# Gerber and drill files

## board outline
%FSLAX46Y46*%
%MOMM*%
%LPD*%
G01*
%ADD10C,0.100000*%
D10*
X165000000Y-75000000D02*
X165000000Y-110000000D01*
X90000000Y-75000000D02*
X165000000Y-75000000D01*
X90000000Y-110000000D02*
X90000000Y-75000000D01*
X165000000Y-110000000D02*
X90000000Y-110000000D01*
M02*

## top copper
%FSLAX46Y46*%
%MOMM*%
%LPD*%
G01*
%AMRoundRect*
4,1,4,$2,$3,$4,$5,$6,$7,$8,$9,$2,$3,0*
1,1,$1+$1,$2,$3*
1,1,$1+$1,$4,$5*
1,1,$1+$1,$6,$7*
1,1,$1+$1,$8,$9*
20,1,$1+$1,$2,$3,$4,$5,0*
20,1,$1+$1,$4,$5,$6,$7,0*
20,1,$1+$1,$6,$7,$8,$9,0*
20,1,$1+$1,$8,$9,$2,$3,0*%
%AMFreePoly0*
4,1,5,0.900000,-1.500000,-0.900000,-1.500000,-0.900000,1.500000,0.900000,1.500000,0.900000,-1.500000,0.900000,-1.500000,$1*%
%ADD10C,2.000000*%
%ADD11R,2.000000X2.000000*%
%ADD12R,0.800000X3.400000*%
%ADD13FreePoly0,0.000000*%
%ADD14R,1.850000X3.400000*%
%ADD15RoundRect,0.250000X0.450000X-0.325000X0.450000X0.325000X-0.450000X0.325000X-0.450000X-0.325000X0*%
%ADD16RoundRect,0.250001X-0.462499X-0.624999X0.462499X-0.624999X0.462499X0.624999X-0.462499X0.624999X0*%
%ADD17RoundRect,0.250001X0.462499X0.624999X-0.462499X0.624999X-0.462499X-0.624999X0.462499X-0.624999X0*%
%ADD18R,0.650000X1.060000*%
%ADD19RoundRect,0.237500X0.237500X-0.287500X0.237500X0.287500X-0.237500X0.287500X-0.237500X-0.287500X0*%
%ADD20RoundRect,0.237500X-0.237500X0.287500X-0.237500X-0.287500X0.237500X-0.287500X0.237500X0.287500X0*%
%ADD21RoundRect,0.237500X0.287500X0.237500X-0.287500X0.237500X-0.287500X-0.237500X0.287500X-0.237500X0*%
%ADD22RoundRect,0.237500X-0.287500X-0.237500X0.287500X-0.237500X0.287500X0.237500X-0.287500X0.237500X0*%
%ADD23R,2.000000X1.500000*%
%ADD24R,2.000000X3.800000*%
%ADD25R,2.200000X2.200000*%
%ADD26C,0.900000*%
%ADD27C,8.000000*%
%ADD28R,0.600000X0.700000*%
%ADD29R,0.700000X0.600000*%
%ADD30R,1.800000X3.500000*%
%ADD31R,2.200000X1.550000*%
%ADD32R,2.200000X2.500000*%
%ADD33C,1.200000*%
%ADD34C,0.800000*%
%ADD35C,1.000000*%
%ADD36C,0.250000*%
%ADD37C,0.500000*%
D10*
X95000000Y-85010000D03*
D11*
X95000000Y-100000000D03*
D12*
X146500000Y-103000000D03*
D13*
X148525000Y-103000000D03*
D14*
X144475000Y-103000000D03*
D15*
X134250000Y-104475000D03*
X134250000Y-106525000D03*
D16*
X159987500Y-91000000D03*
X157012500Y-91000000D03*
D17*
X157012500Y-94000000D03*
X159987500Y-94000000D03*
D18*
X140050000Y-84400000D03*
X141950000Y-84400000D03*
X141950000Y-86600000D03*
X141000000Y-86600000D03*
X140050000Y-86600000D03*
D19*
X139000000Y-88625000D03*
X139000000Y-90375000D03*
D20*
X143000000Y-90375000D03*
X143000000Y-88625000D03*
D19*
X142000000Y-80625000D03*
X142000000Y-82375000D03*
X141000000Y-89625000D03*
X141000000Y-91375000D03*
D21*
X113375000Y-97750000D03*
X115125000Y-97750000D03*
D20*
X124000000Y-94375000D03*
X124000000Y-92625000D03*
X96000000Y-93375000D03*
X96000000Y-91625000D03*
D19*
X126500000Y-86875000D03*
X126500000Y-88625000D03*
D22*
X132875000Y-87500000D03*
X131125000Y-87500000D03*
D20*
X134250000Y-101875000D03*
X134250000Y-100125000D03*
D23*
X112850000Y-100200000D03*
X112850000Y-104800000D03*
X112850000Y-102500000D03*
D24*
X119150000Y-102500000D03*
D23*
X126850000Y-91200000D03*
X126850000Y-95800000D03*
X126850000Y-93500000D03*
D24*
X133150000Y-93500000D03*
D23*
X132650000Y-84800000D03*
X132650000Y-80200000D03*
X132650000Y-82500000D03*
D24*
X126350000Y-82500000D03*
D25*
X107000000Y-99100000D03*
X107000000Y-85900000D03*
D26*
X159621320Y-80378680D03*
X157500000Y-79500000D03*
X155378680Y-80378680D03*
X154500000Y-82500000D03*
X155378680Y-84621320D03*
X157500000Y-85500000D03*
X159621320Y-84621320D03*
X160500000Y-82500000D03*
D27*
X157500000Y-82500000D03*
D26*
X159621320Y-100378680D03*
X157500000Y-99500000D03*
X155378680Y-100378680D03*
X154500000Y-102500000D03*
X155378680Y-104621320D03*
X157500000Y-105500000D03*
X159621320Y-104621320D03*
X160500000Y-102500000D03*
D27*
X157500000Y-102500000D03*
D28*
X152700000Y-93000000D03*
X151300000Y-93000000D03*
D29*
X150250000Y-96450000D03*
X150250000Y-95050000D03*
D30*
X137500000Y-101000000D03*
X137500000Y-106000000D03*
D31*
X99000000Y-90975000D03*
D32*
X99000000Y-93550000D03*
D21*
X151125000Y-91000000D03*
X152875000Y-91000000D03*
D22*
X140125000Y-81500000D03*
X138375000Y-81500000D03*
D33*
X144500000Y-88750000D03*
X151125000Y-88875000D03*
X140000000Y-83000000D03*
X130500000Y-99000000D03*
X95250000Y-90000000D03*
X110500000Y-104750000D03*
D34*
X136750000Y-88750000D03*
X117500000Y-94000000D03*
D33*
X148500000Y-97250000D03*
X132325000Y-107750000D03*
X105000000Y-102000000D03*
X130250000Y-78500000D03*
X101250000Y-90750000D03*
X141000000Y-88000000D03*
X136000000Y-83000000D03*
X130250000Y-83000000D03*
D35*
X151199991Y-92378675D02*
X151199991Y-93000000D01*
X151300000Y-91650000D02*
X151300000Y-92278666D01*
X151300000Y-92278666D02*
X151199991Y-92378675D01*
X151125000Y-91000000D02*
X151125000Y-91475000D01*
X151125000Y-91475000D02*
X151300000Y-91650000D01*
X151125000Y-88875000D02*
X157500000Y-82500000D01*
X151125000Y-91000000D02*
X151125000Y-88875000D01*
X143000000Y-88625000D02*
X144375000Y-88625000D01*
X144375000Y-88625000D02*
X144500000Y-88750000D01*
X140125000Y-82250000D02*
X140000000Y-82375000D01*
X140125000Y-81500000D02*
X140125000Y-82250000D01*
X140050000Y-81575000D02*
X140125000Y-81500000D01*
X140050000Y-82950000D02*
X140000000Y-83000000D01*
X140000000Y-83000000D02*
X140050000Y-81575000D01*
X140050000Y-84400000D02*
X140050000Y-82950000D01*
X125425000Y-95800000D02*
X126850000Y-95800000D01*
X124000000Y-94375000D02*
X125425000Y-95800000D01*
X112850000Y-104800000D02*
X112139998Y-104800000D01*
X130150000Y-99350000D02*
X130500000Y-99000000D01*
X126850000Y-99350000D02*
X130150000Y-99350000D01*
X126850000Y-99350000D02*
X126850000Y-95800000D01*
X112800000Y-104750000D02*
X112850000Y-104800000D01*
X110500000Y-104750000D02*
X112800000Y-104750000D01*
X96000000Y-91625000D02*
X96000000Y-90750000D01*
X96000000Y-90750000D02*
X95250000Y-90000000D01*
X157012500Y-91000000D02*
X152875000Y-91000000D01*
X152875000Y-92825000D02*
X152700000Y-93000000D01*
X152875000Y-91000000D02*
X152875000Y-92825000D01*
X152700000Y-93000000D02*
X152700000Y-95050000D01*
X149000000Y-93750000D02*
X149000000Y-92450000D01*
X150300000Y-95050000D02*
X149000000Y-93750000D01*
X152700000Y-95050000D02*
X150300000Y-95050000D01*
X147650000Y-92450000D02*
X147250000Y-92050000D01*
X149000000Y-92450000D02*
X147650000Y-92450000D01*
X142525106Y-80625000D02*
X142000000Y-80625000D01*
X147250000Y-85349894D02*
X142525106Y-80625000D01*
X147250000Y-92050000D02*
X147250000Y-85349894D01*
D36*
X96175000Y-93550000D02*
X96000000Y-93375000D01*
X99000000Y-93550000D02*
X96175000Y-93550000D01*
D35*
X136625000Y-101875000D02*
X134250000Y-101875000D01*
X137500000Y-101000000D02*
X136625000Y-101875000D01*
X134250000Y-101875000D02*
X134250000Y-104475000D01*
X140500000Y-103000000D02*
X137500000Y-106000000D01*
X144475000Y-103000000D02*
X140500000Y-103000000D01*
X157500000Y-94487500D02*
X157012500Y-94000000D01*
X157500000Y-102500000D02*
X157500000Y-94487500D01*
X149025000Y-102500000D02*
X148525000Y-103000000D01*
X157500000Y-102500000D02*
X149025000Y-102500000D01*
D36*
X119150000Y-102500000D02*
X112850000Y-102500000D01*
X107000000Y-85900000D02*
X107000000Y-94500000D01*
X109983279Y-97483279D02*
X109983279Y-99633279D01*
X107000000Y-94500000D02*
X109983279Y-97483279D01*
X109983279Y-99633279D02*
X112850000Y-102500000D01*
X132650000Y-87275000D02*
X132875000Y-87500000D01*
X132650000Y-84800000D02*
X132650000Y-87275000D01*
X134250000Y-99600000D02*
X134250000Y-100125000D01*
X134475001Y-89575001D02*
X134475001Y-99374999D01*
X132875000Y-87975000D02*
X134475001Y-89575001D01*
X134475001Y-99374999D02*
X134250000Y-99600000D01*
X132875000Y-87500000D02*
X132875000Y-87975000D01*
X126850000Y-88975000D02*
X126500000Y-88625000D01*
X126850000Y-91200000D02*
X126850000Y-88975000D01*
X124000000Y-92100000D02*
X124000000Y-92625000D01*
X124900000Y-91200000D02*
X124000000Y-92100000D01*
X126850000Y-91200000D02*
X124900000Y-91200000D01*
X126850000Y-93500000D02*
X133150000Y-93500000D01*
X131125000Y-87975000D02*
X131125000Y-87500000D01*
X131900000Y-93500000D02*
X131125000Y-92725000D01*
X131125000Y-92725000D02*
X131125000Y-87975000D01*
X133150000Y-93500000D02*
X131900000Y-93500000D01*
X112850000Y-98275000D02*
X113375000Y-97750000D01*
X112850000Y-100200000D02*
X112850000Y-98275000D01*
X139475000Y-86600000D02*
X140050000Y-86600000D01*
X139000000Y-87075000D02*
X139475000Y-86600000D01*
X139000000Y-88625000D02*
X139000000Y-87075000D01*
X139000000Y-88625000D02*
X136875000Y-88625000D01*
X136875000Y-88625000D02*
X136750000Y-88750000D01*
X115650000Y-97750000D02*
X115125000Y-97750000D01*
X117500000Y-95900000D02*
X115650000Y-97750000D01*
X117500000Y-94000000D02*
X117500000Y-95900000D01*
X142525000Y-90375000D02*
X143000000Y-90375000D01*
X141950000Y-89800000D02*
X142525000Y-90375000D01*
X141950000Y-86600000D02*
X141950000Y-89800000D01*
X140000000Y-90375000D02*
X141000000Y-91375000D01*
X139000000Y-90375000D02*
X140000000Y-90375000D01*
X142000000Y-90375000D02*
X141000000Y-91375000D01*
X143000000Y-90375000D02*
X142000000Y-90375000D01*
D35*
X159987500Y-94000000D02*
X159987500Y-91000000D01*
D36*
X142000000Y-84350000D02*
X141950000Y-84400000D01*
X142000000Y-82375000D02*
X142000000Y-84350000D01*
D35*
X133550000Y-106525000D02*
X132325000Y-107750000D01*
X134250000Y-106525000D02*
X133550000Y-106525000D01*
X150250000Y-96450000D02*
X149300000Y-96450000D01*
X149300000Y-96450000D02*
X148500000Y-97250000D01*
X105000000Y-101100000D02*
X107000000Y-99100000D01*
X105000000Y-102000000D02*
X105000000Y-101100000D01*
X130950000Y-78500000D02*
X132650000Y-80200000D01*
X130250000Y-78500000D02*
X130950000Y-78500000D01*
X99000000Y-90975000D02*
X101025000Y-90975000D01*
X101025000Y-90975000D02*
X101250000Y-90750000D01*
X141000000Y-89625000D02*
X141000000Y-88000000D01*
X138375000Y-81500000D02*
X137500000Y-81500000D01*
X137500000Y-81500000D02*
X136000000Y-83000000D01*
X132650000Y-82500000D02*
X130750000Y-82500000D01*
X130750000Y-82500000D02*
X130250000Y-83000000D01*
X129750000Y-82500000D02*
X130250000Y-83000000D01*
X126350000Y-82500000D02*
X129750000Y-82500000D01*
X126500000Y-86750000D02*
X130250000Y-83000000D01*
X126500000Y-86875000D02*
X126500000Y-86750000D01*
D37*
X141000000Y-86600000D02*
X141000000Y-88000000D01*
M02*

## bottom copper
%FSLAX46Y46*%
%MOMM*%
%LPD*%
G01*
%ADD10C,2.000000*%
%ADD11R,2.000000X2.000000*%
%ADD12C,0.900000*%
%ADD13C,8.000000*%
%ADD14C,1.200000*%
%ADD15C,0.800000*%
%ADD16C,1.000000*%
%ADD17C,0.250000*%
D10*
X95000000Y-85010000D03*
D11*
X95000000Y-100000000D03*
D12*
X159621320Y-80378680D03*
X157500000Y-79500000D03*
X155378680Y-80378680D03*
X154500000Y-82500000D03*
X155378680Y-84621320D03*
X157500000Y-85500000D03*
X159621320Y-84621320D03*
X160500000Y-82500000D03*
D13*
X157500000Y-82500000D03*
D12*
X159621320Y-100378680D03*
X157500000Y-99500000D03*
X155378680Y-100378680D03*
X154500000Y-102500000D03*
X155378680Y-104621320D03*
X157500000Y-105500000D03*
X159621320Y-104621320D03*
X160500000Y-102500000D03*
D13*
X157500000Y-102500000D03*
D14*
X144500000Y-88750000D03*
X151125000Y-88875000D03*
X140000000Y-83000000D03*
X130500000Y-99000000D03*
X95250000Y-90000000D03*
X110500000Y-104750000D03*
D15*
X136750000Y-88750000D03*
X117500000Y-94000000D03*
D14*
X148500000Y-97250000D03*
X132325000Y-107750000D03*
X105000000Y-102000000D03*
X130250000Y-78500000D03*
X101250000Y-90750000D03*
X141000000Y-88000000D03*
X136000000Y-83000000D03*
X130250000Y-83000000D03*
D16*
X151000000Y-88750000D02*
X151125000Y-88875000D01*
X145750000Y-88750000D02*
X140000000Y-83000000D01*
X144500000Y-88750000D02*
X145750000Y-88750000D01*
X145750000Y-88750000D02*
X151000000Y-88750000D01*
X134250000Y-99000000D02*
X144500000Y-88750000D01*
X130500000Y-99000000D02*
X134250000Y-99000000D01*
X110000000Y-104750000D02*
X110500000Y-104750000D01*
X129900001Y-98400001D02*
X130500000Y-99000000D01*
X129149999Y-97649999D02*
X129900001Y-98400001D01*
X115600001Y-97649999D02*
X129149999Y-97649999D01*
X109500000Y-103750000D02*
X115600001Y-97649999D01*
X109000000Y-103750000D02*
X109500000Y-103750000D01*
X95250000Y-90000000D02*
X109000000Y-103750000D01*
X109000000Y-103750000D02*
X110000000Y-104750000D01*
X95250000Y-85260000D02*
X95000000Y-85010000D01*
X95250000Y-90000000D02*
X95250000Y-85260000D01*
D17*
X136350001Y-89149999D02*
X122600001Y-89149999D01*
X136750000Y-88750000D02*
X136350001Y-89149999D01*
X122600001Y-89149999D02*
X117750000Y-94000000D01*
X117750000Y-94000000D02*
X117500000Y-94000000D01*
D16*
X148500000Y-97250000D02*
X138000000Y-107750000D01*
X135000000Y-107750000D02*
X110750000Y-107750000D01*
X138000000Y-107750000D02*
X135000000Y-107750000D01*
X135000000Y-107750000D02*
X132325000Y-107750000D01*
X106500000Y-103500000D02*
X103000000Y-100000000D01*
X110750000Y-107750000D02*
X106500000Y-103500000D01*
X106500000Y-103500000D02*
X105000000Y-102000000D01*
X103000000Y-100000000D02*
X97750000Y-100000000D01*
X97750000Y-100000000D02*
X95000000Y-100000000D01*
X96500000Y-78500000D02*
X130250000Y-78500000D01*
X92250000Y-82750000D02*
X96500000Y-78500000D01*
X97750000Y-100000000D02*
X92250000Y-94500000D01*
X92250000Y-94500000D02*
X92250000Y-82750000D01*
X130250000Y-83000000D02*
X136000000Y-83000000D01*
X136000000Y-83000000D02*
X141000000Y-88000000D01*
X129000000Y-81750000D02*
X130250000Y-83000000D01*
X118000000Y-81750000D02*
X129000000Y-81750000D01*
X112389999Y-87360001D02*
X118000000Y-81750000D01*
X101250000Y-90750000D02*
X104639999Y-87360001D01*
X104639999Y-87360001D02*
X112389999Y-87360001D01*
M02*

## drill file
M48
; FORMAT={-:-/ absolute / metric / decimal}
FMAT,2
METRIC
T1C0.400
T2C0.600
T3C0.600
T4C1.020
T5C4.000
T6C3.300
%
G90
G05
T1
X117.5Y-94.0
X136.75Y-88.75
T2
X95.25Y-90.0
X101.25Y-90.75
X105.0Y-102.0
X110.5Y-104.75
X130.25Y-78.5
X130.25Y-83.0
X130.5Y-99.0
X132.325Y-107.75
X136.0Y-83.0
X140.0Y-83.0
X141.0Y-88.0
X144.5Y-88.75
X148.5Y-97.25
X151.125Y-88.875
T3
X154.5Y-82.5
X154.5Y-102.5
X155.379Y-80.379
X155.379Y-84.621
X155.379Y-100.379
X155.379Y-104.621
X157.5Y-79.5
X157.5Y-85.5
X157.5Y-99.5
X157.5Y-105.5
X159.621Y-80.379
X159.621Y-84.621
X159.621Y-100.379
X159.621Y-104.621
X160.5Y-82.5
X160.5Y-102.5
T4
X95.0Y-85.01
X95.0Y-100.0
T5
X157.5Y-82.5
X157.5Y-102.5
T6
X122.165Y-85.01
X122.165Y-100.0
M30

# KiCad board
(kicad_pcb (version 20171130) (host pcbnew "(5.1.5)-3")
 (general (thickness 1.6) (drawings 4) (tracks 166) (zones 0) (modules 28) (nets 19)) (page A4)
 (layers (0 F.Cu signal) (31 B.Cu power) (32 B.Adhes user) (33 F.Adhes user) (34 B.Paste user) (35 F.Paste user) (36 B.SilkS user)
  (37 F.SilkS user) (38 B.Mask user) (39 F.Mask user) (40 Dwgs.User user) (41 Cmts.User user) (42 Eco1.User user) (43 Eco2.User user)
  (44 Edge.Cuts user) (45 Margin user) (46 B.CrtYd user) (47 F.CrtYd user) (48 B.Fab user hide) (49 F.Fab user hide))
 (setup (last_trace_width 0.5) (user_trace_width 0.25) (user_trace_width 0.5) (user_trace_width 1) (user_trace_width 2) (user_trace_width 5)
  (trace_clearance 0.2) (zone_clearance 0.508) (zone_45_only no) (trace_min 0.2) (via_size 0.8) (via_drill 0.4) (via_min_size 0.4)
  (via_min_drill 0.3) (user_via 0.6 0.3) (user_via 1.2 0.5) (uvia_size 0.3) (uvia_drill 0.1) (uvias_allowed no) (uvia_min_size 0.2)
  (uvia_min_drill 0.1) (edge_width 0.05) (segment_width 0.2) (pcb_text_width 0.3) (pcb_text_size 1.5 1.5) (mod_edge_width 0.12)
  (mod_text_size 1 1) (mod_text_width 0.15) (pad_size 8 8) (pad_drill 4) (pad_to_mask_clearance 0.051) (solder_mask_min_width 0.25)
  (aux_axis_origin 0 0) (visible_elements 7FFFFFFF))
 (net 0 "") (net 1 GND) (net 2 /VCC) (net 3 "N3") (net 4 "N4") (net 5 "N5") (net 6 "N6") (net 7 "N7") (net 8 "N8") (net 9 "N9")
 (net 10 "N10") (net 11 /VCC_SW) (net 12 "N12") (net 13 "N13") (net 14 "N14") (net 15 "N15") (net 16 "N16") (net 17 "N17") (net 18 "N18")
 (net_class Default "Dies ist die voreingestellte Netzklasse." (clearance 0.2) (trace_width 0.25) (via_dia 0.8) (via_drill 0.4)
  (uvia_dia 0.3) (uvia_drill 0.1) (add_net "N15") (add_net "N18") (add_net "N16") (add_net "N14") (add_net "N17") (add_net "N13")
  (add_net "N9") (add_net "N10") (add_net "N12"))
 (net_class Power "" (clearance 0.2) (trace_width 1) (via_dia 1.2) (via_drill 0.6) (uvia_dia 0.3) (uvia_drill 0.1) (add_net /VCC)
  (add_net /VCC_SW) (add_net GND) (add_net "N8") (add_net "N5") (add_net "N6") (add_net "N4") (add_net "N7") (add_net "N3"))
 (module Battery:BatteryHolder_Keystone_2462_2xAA (layer B.Cu) (at 95 100)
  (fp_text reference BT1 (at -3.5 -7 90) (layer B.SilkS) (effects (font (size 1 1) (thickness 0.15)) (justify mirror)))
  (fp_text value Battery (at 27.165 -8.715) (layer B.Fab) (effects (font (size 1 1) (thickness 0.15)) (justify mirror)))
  (pad "" np_thru_hole circle (at 27.165 0) (size 3.3 3.3) (drill 3.3) (layers *.Cu *.Mask))
  (pad "" np_thru_hole circle (at 27.165 -14.99) (size 3.3 3.3) (drill 3.3) (layers *.Cu *.Mask))
  (pad 2 thru_hole circle (at 0 -14.99) (size 2 2) (drill 1.02) (layers *.Cu *.Mask) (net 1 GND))
  (pad 1 thru_hole rect (at 0 0) (size 2 2) (drill 1.02) (layers *.Cu *.Mask) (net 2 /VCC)))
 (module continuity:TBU (layer F.Cu) (at 146.5 103)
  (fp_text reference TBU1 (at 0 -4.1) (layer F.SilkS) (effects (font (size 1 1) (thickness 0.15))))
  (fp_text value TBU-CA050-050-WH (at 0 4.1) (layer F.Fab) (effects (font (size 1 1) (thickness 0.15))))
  (pad 2 smd rect (at 0 0) (size 0.8 3.4) (layers F.Cu F.Paste F.Mask) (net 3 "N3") (zone_connect 2))
  (pad 3 smd custom (at 2.025 0) (size 1.8 3) (layers F.Cu F.Paste F.Mask) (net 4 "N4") (zone_connect 2)
   (options (clearance outline) (anchor rect)) (primitives))
  (pad 1 smd rect (at -2.025 0) (size 1.85 3.4) (layers F.Cu F.Paste F.Mask) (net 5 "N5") (zone_connect 2)))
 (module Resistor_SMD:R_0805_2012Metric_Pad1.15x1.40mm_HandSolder (layer F.Cu) (at 134.25 105.5 90)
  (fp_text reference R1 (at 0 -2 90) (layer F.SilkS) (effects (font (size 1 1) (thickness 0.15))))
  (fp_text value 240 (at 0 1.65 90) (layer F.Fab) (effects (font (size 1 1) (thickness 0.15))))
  (pad 2 smd roundrect (at 1.025 0 90) (size 1.15 1.4) (layers F.Cu F.Paste F.Mask) (roundrect_rratio 0.217391) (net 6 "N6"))
  (pad 1 smd roundrect (at -1.025 0 90) (size 1.15 1.4) (layers F.Cu F.Paste F.Mask) (roundrect_rratio 0.217391) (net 2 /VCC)))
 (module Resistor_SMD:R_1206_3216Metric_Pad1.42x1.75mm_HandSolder (layer F.Cu) (at 158.5 91)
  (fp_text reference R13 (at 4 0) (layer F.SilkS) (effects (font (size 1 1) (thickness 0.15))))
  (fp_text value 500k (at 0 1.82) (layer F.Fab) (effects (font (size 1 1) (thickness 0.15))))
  (pad 2 smd roundrect (at 1.4875 0) (size 1.425 1.75) (layers F.Cu F.Paste F.Mask) (roundrect_rratio 0.175439) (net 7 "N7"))
  (pad 1 smd roundrect (at -1.4875 0) (size 1.425 1.75) (layers F.Cu F.Paste F.Mask) (roundrect_rratio 0.175439) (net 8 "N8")))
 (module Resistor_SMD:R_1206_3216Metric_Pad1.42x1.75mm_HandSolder (layer F.Cu) (at 158.5 94 180)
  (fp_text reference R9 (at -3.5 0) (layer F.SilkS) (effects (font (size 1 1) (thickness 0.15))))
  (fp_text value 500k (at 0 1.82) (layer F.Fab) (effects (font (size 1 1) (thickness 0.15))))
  (pad 2 smd roundrect (at 1.4875 0 180) (size 1.425 1.75) (layers F.Cu F.Paste F.Mask) (roundrect_rratio 0.175439) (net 4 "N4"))
  (pad 1 smd roundrect (at -1.4875 0 180) (size 1.425 1.75) (layers F.Cu F.Paste F.Mask) (roundrect_rratio 0.175439) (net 7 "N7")))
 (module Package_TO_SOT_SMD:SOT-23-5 (layer F.Cu) (at 141 85.5 90)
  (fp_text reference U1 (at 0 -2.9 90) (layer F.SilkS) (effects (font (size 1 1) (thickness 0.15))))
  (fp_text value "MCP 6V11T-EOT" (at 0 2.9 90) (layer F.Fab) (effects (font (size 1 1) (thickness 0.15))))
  (pad 5 smd rect (at 1.1 -0.95 90) (size 1.06 0.65) (layers F.Cu F.Paste F.Mask) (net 1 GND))
  (pad 4 smd rect (at 1.1 0.95 90) (size 1.06 0.65) (layers F.Cu F.Paste F.Mask) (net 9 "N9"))
  (pad 3 smd rect (at -1.1 0.95 90) (size 1.06 0.65) (layers F.Cu F.Paste F.Mask) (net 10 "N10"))
  (pad 2 smd rect (at -1.1 0 90) (size 1.06 0.65) (layers F.Cu F.Paste F.Mask) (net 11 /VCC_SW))
  (pad 1 smd rect (at -1.1 -0.95 90) (size 1.06 0.65) (layers F.Cu F.Paste F.Mask) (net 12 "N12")))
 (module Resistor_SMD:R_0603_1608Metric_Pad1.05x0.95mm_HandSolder (layer F.Cu) (at 139 89.5 90)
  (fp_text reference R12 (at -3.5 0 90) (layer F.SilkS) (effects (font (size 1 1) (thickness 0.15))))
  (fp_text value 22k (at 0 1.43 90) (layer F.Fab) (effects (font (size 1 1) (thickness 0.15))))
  (pad 2 smd roundrect (at 0.875 0 90) (size 1.05 0.95) (layers F.Cu F.Paste F.Mask) (roundrect_rratio 0.25) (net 12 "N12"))
  (pad 1 smd roundrect (at -0.875 0 90) (size 1.05 0.95) (layers F.Cu F.Paste F.Mask) (roundrect_rratio 0.25) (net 10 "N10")))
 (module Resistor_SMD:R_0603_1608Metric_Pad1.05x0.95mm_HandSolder (layer F.Cu) (at 143 89.5 270)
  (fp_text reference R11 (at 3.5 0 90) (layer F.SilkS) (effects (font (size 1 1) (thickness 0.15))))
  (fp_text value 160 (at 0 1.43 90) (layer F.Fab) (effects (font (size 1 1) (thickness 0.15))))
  (pad 2 smd roundrect (at 0.875 0 270) (size 1.05 0.95) (layers F.Cu F.Paste F.Mask) (roundrect_rratio 0.25) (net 10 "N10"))
  (pad 1 smd roundrect (at -0.875 0 270) (size 1.05 0.95) (layers F.Cu F.Paste F.Mask) (roundrect_rratio 0.25) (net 1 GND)))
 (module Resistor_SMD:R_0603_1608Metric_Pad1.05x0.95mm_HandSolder (layer F.Cu) (at 142 81.5 90)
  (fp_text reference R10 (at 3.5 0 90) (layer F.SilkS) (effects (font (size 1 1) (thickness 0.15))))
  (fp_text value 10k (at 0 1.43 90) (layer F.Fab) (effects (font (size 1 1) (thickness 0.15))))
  (pad 2 smd roundrect (at 0.875 0 90) (size 1.05 0.95) (layers F.Cu F.Paste F.Mask) (roundrect_rratio 0.25) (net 8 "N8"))
  (pad 1 smd roundrect (at -0.875 0 90) (size 1.05 0.95) (layers F.Cu F.Paste F.Mask) (roundrect_rratio 0.25) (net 9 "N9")))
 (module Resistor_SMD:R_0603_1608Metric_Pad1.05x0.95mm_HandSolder (layer F.Cu) (at 141 90.5 90)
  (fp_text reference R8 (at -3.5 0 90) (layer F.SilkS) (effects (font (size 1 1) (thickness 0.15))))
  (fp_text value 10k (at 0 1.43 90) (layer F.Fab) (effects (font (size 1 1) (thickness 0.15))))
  (pad 2 smd roundrect (at 0.875 0 90) (size 1.05 0.95) (layers F.Cu F.Paste F.Mask) (roundrect_rratio 0.25) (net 11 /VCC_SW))
  (pad 1 smd roundrect (at -0.875 0 90) (size 1.05 0.95) (layers F.Cu F.Paste F.Mask) (roundrect_rratio 0.25) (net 10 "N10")))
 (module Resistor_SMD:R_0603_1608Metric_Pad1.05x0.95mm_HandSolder (layer F.Cu) (at 114.25 97.75 180)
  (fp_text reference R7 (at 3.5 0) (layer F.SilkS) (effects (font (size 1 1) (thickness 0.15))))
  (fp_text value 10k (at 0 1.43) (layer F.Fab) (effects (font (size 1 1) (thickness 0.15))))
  (pad 2 smd roundrect (at 0.875 0 180) (size 1.05 0.95) (layers F.Cu F.Paste F.Mask) (roundrect_rratio 0.25) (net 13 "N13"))
  (pad 1 smd roundrect (at -0.875 0 180) (size 1.05 0.95) (layers F.Cu F.Paste F.Mask) (roundrect_rratio 0.25) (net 12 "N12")))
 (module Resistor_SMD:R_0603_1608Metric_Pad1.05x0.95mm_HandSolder (layer F.Cu) (at 124 93.5 270)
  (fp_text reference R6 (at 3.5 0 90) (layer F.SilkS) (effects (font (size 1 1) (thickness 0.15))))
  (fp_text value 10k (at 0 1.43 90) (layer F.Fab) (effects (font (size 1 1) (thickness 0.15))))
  (pad 2 smd roundrect (at 0.875 0 270) (size 1.05 0.95) (layers F.Cu F.Paste F.Mask) (roundrect_rratio 0.25) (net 1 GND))
  (pad 1 smd roundrect (at -0.875 0 270) (size 1.05 0.95) (layers F.Cu F.Paste F.Mask) (roundrect_rratio 0.25) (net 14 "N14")))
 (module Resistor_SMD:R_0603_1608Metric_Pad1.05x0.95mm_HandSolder (layer F.Cu) (at 96 92.5 270)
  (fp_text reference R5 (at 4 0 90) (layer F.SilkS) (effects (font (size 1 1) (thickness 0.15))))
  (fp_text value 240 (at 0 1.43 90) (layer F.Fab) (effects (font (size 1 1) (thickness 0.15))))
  (pad 2 smd roundrect (at 0.875 0 270) (size 1.05 0.95) (layers F.Cu F.Paste F.Mask) (roundrect_rratio 0.25) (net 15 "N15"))
  (pad 1 smd roundrect (at -0.875 0 270) (size 1.05 0.95) (layers F.Cu F.Paste F.Mask) (roundrect_rratio 0.25) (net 1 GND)))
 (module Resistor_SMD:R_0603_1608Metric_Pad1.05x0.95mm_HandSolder (layer F.Cu) (at 126.5 87.75 90)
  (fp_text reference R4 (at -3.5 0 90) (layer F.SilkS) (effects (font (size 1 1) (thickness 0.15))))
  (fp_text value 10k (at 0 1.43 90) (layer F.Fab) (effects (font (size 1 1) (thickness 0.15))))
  (pad 2 smd roundrect (at 0.875 0 90) (size 1.05 0.95) (layers F.Cu F.Paste F.Mask) (roundrect_rratio 0.25) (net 11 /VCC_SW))
  (pad 1 smd roundrect (at -0.875 0 90) (size 1.05 0.95) (layers F.Cu F.Paste F.Mask) (roundrect_rratio 0.25) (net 14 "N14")))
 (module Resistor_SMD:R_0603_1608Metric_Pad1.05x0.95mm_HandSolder (layer F.Cu) (at 132 87.5)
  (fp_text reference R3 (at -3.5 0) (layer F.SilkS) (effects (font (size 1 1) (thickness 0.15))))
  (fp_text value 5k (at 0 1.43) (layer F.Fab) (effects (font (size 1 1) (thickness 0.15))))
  (pad 2 smd roundrect (at 0.875 0) (size 1.05 0.95) (layers F.Cu F.Paste F.Mask) (roundrect_rratio 0.25) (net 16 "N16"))
  (pad 1 smd roundrect (at -0.875 0) (size 1.05 0.95) (layers F.Cu F.Paste F.Mask) (roundrect_rratio 0.25) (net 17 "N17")))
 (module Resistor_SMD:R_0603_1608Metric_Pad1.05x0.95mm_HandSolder (layer F.Cu) (at 134.25 101 270)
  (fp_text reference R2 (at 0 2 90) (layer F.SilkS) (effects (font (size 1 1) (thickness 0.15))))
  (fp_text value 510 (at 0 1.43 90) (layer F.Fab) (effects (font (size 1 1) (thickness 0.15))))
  (pad 2 smd roundrect (at 0.875 0 270) (size 1.05 0.95) (layers F.Cu F.Paste F.Mask) (roundrect_rratio 0.25) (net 6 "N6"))
  (pad 1 smd roundrect (at -0.875 0 270) (size 1.05 0.95) (layers F.Cu F.Paste F.Mask) (roundrect_rratio 0.25) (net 16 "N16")))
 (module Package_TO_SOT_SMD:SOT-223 (layer F.Cu) (at 116 102.5)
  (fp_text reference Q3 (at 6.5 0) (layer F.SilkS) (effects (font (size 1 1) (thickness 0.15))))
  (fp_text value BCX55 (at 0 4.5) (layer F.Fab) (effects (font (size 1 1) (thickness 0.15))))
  (pad 1 smd rect (at -3.15 -2.3) (size 2 1.5) (layers F.Cu F.Paste F.Mask) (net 13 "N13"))
  (pad 3 smd rect (at -3.15 2.3) (size 2 1.5) (layers F.Cu F.Paste F.Mask) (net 1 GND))
  (pad 2 smd rect (at -3.15 0) (size 2 1.5) (layers F.Cu F.Paste F.Mask) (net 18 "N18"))
  (pad 4 smd rect (at 3.15 0) (size 2 3.8) (layers F.Cu F.Paste F.Mask) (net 18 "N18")))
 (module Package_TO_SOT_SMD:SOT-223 (layer F.Cu) (at 130 93.5)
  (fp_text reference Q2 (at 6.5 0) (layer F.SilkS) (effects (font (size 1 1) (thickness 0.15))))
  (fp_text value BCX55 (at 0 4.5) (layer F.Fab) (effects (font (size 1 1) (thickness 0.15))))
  (pad 1 smd rect (at -3.15 -2.3) (size 2 1.5) (layers F.Cu F.Paste F.Mask) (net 14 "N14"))
  (pad 3 smd rect (at -3.15 2.3) (size 2 1.5) (layers F.Cu F.Paste F.Mask) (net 1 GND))
  (pad 2 smd rect (at -3.15 0) (size 2 1.5) (layers F.Cu F.Paste F.Mask) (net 17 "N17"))
  (pad 4 smd rect (at 3.15 0) (size 2 3.8) (layers F.Cu F.Paste F.Mask) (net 17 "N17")))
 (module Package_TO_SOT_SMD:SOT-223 (layer F.Cu) (at 129.5 82.5 180)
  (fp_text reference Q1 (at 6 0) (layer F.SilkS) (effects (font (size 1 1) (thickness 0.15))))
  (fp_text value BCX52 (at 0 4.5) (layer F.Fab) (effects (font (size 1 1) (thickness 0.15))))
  (pad 1 smd rect (at -3.15 -2.3 180) (size 2 1.5) (layers F.Cu F.Paste F.Mask) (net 16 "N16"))
  (pad 3 smd rect (at -3.15 2.3 180) (size 2 1.5) (layers F.Cu F.Paste F.Mask) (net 2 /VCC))
  (pad 2 smd rect (at -3.15 0 180) (size 2 1.5) (layers F.Cu F.Paste F.Mask) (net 11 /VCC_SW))
  (pad 4 smd rect (at 3.15 0 180) (size 2 3.8) (layers F.Cu F.Paste F.Mask) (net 11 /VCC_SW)))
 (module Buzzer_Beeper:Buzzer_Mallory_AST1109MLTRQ (layer F.Cu) (at 107 92.5 90)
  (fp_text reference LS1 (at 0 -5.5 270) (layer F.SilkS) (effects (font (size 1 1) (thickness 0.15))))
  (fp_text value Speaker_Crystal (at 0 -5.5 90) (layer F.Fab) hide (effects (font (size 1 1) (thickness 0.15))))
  (pad 1 smd rect (at -6.6 0 90) (size 2.2 2.2) (layers F.Cu F.Paste F.Mask) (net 2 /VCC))
  (pad 2 smd rect (at 6.6 0 90) (size 2.2 2.2) (layers F.Cu F.Paste F.Mask) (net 18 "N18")))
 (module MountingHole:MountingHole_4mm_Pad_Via (layer F.Cu) (at 157.5 82.5)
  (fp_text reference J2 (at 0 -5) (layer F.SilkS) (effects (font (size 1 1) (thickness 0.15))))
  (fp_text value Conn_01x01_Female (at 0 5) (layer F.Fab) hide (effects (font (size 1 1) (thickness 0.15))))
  (pad 1 thru_hole circle (at 2.12132 -2.12132) (size 0.9 0.9) (drill 0.6) (layers *.Cu *.Mask) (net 1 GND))
  (pad 1 thru_hole circle (at 0 -3) (size 0.9 0.9) (drill 0.6) (layers *.Cu *.Mask) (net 1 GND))
  (pad 1 thru_hole circle (at -2.12132 -2.12132) (size 0.9 0.9) (drill 0.6) (layers *.Cu *.Mask) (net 1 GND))
  (pad 1 thru_hole circle (at -3 0) (size 0.9 0.9) (drill 0.6) (layers *.Cu *.Mask) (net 1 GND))
  (pad 1 thru_hole circle (at -2.12132 2.12132) (size 0.9 0.9) (drill 0.6) (layers *.Cu *.Mask) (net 1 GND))
  (pad 1 thru_hole circle (at 0 3) (size 0.9 0.9) (drill 0.6) (layers *.Cu *.Mask) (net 1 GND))
  (pad 1 thru_hole circle (at 2.12132 2.12132) (size 0.9 0.9) (drill 0.6) (layers *.Cu *.Mask) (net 1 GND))
  (pad 1 thru_hole circle (at 3 0) (size 0.9 0.9) (drill 0.6) (layers *.Cu *.Mask) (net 1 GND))
  (pad 1 thru_hole circle (at 0 0) (size 8 8) (drill 4) (layers *.Cu *.Mask) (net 1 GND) (zone_connect 2)))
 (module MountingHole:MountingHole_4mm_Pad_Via (layer F.Cu) (at 157.5 102.5)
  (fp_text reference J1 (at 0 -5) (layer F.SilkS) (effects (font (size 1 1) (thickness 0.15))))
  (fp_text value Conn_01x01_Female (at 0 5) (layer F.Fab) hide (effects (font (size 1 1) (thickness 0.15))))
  (pad 1 thru_hole circle (at 2.12132 -2.12132) (size 0.9 0.9) (drill 0.6) (layers *.Cu *.Mask) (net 4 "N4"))
  (pad 1 thru_hole circle (at 0 -3) (size 0.9 0.9) (drill 0.6) (layers *.Cu *.Mask) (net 4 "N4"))
  (pad 1 thru_hole circle (at -2.12132 -2.12132) (size 0.9 0.9) (drill 0.6) (layers *.Cu *.Mask) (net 4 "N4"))
  (pad 1 thru_hole circle (at -3 0) (size 0.9 0.9) (drill 0.6) (layers *.Cu *.Mask) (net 4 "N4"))
  (pad 1 thru_hole circle (at -2.12132 2.12132) (size 0.9 0.9) (drill 0.6) (layers *.Cu *.Mask) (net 4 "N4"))
  (pad 1 thru_hole circle (at 0 3) (size 0.9 0.9) (drill 0.6) (layers *.Cu *.Mask) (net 4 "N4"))
  (pad 1 thru_hole circle (at 2.12132 2.12132) (size 0.9 0.9) (drill 0.6) (layers *.Cu *.Mask) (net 4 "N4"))
  (pad 1 thru_hole circle (at 3 0) (size 0.9 0.9) (drill 0.6) (layers *.Cu *.Mask) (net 4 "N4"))
  (pad 1 thru_hole circle (at 0 0) (size 8 8) (drill 4) (layers *.Cu *.Mask) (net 4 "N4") (zone_connect 2)))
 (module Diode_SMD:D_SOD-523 (layer F.Cu) (at 152 93 180)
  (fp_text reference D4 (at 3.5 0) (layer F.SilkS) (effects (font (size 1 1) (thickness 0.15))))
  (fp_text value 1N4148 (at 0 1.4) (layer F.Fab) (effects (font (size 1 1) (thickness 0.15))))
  (pad 1 smd rect (at -0.7 0) (size 0.6 0.7) (layers F.Cu F.Paste F.Mask) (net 8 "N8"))
  (pad 2 smd rect (at 0.7 0) (size 0.6 0.7) (layers F.Cu F.Paste F.Mask) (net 1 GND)))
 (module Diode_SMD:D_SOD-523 (layer F.Cu) (at 150.25 95.75 90)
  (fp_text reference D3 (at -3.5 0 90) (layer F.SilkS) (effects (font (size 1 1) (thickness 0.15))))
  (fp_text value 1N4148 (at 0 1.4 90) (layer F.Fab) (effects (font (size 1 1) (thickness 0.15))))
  (pad 1 smd rect (at -0.7 0 270) (size 0.6 0.7) (layers F.Cu F.Paste F.Mask) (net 2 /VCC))
  (pad 2 smd rect (at 0.7 0 270) (size 0.6 0.7) (layers F.Cu F.Paste F.Mask) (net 8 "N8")))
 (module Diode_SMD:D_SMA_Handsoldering (layer F.Cu) (at 137.5 103.5 90)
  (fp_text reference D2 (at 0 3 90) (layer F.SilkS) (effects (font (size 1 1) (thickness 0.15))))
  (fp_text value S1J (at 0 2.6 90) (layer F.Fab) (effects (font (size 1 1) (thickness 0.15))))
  (pad 2 smd rect (at 2.5 0 90) (size 3.5 1.8) (layers F.Cu F.Paste F.Mask) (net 6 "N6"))
  (pad 1 smd rect (at -2.5 0 90) (size 3.5 1.8) (layers F.Cu F.Paste F.Mask) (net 5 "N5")))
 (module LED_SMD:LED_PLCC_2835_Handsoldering (layer F.Cu) (at 99 92.5 90)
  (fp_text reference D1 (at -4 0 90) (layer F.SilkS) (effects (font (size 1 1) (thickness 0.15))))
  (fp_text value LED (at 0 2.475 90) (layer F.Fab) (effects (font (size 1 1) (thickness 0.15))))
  (pad 2 smd rect (at 1.525 0 90) (size 1.55 2.2) (layers F.Cu F.Paste F.Mask) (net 11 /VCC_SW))
  (pad 1 smd rect (at -1.05 0 90) (size 2.5 2.2) (layers F.Cu F.Paste F.Mask) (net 15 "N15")))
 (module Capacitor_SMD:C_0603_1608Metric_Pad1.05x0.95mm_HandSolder (layer F.Cu) (at 152 91 180)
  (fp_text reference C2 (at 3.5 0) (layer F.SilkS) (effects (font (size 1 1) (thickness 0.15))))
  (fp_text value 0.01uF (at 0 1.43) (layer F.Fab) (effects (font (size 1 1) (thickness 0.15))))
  (pad 2 smd roundrect (at 0.875 0 180) (size 1.05 0.95) (layers F.Cu F.Paste F.Mask) (roundrect_rratio 0.25) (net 1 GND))
  (pad 1 smd roundrect (at -0.875 0 180) (size 1.05 0.95) (layers F.Cu F.Paste F.Mask) (roundrect_rratio 0.25) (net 8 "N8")))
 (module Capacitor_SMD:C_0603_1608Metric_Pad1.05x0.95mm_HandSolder (layer F.Cu) (at 139.25 81.5)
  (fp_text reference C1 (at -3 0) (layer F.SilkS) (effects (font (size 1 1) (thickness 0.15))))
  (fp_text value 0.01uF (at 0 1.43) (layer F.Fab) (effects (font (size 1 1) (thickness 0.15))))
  (pad 2 smd roundrect (at 0.875 0) (size 1.05 0.95) (layers F.Cu F.Paste F.Mask) (roundrect_rratio 0.25) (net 1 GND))
  (pad 1 smd roundrect (at -0.875 0) (size 1.05 0.95) (layers F.Cu F.Paste F.Mask) (roundrect_rratio 0.25) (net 11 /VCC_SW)))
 (gr_line (start 165 75) (end 165 110) (layer Edge.Cuts) (width 0.1))
 (gr_line (start 90 75) (end 165 75) (layer Edge.Cuts) (width 0.1))
 (gr_line (start 90 110) (end 90 75) (layer Edge.Cuts) (width 0.1))
 (gr_line (start 165 110) (end 90 110) (layer Edge.Cuts) (width 0.1))
 (segment (start 151.199991 92.378675) (end 151.199991 93) (width 1) (layer F.Cu) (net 1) (status 20))
 (segment (start 151.3 91.65) (end 151.3 92.278666) (width 1) (layer F.Cu) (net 1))
 (segment (start 151.3 92.278666) (end 151.199991 92.378675) (width 1) (layer F.Cu) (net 1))
 (segment (start 151.125 91) (end 151.125 91.475) (width 1) (layer F.Cu) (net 1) (status 10))
 (segment (start 151.125 91.475) (end 151.3 91.65) (width 1) (layer F.Cu) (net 1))
 (segment (start 151.125 88.875) (end 157.5 82.5) (width 1) (layer F.Cu) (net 1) (status 20))
 (segment (start 151.125 91) (end 151.125 88.875) (width 1) (layer F.Cu) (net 1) (status 10))
 (via (at 144.5 88.75) (size 1.2) (drill 0.6) (layers F.Cu B.Cu) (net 1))
 (segment (start 143 88.625) (end 144.375 88.625) (width 1) (layer F.Cu) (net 1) (status 10))
 (segment (start 144.375 88.625) (end 144.5 88.75) (width 1) (layer F.Cu) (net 1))
 (via (at 151.125 88.875) (size 1.2) (drill 0.6) (layers F.Cu B.Cu) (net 1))
 (segment (start 151 88.75) (end 151.125 88.875) (width 1) (layer B.Cu) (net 1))
 (segment (start 140.125 82.25) (end 140 82.375) (width 1) (layer F.Cu) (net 1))
 (segment (start 140.125 81.5) (end 140.125 82.25) (width 1) (layer F.Cu) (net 1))
 (segment (start 140.05 81.575) (end 140.125 81.5) (width 1) (layer F.Cu) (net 1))
 (segment (start 140.05 82.95) (end 140 83) (width 1) (layer F.Cu) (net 1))
 (via (at 140 83) (size 1.2) (drill 0.6) (layers F.Cu B.Cu) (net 1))
 (segment (start 140 83) (end 140.05 81.575) (width 1) (layer F.Cu) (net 1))
 (segment (start 140.05 84.4) (end 140.05 82.95) (width 1) (layer F.Cu) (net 1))
 (segment (start 145.75 88.75) (end 140 83) (width 1) (layer B.Cu) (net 1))
 (segment (start 144.5 88.75) (end 145.75 88.75) (width 1) (layer B.Cu) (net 1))
 (segment (start 145.75 88.75) (end 151 88.75) (width 1) (layer B.Cu) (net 1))
 (segment (start 125.425 95.8) (end 126.85 95.8) (width 1) (layer F.Cu) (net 1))
 (segment (start 124 94.375) (end 125.425 95.8) (width 1) (layer F.Cu) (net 1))
 (segment (start 112.85 104.8) (end 112.139998 104.8) (width 1) (layer F.Cu) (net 1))
 (via (at 130.5 99) (size 1.2) (drill 0.6) (layers F.Cu B.Cu) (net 1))
 (segment (start 130.15 99.35) (end 130.5 99) (width 1) (layer F.Cu) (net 1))
 (segment (start 126.85 99.35) (end 130.15 99.35) (width 1) (layer F.Cu) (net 1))
 (segment (start 126.85 99.35) (end 126.85 95.8) (width 1) (layer F.Cu) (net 1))
 (segment (start 134.25 99) (end 144.5 88.75) (width 1) (layer B.Cu) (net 1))
 (segment (start 130.5 99) (end 134.25 99) (width 1) (layer B.Cu) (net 1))
 (via (at 95.25 90) (size 1.2) (drill 0.6) (layers F.Cu B.Cu) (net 1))
 (via (at 110.5 104.75) (size 1.2) (drill 0.6) (layers F.Cu B.Cu) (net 1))
 (segment (start 110 104.75) (end 110.5 104.75) (width 1) (layer B.Cu) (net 1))
 (segment (start 112.8 104.75) (end 112.85 104.8) (width 1) (layer F.Cu) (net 1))
 (segment (start 110.5 104.75) (end 112.8 104.75) (width 1) (layer F.Cu) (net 1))
 (segment (start 129.900001 98.400001) (end 130.5 99) (width 1) (layer B.Cu) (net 1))
 (segment (start 129.149999 97.649999) (end 129.900001 98.400001) (width 1) (layer B.Cu) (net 1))
 (segment (start 115.600001 97.649999) (end 129.149999 97.649999) (width 1) (layer B.Cu) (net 1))
 (segment (start 109.5 103.75) (end 115.600001 97.649999) (width 1) (layer B.Cu) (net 1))
 (segment (start 109 103.75) (end 109.5 103.75) (width 1) (layer B.Cu) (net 1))
 (segment (start 95.25 90) (end 109 103.75) (width 1) (layer B.Cu) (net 1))
 (segment (start 109 103.75) (end 110 104.75) (width 1) (layer B.Cu) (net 1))
 (segment (start 96 91.625) (end 96 90.75) (width 1) (layer F.Cu) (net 1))
 (segment (start 96 90.75) (end 95.25 90) (width 1) (layer F.Cu) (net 1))
 (segment (start 95.25 85.26) (end 95 85.01) (width 1) (layer B.Cu) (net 1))
 (segment (start 95.25 90) (end 95.25 85.26) (width 1) (layer B.Cu) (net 1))
 (segment (start 157.0125 91) (end 152.875 91) (width 1) (layer F.Cu) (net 8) (status 30))
 (segment (start 152.875 92.825) (end 152.7 93) (width 1) (layer F.Cu) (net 8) (status 30))
 (segment (start 152.875 91) (end 152.875 92.825) (width 1) (layer F.Cu) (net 8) (status 30))
 (segment (start 152.7 93) (end 152.7 95.05) (width 1) (layer F.Cu) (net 8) (status 10))
 (segment (start 149 93.75) (end 149 92.45) (width 1) (layer F.Cu) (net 8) (status 20))
 (segment (start 150.3 95.05) (end 149 93.75) (width 1) (layer F.Cu) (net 8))
 (segment (start 152.7 95.05) (end 150.3 95.05) (width 1) (layer F.Cu) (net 8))
 (segment (start 147.65 92.45) (end 147.25 92.05) (width 1) (layer F.Cu) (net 8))
 (segment (start 149 92.45) (end 147.65 92.45) (width 1) (layer F.Cu) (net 8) (status 10))
 (segment (start 142.525106 80.625) (end 142 80.625) (width 1) (layer F.Cu) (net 8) (status 20))
 (segment (start 147.25 85.349894) (end 142.525106 80.625) (width 1) (layer F.Cu) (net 8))
 (segment (start 147.25 92.05) (end 147.25 85.349894) (width 1) (layer F.Cu) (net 8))
 (segment (start 96.175 93.55) (end 96 93.375) (width 0.25) (layer F.Cu) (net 15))
 (segment (start 99 93.55) (end 96.175 93.55) (width 0.25) (layer F.Cu) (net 15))
 (segment (start 136.625 101.875) (end 134.25 101.875) (width 1) (layer F.Cu) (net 6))
 (segment (start 137.5 101) (end 136.625 101.875) (width 1) (layer F.Cu) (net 6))
 (segment (start 134.25 101.875) (end 134.25 104.475) (width 1) (layer F.Cu) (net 6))
 (segment (start 140.5 103) (end 137.5 106) (width 1) (layer F.Cu) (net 5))
 (segment (start 144.475 103) (end 140.5 103) (width 1) (layer F.Cu) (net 5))
 (segment (start 157.5 94.4875) (end 157.0125 94) (width 1) (layer F.Cu) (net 4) (status 30))
 (segment (start 157.5 102.5) (end 157.5 94.4875) (width 1) (layer F.Cu) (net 4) (status 30))
 (segment (start 149.025 102.5) (end 148.525 103) (width 1) (layer F.Cu) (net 4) (status 30))
 (segment (start 157.5 102.5) (end 149.025 102.5) (width 1) (layer F.Cu) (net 4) (status 30))
 (segment (start 119.15 102.5) (end 112.85 102.5) (width 0.25) (layer F.Cu) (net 18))
 (segment (start 107 85.9) (end 107 94.5) (width 0.25) (layer F.Cu) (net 18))
 (segment (start 109.983279 97.483279) (end 109.983279 99.633279) (width 0.25) (layer F.Cu) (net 18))
 (segment (start 107 94.5) (end 109.983279 97.483279) (width 0.25) (layer F.Cu) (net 18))
 (segment (start 109.983279 99.633279) (end 112.85 102.5) (width 0.25) (layer F.Cu) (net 18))
 (segment (start 132.65 87.275) (end 132.875 87.5) (width 0.25) (layer F.Cu) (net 16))
 (segment (start 132.65 84.8) (end 132.65 87.275) (width 0.25) (layer F.Cu) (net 16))
 (segment (start 134.25 99.6) (end 134.25 100.125) (width 0.25) (layer F.Cu) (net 16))
 (segment (start 134.475001 89.575001) (end 134.475001 99.374999) (width 0.25) (layer F.Cu) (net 16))
 (segment (start 132.875 87.975) (end 134.475001 89.575001) (width 0.25) (layer F.Cu) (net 16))
 (segment (start 134.475001 99.374999) (end 134.25 99.6) (width 0.25) (layer F.Cu) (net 16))
 (segment (start 132.875 87.5) (end 132.875 87.975) (width 0.25) (layer F.Cu) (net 16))
 (segment (start 126.85 88.975) (end 126.5 88.625) (width 0.25) (layer F.Cu) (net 14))
 (segment (start 126.85 91.2) (end 126.85 88.975) (width 0.25) (layer F.Cu) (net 14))
 (segment (start 124 92.1) (end 124 92.625) (width 0.25) (layer F.Cu) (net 14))
 (segment (start 124.9 91.2) (end 124 92.1) (width 0.25) (layer F.Cu) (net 14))
 (segment (start 126.85 91.2) (end 124.9 91.2) (width 0.25) (layer F.Cu) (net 14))
 (segment (start 126.85 93.5) (end 133.15 93.5) (width 0.25) (layer F.Cu) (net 17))
 (segment (start 131.125 87.975) (end 131.125 87.5) (width 0.25) (layer F.Cu) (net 17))
 (segment (start 131.9 93.5) (end 131.125 92.725) (width 0.25) (layer F.Cu) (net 17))
 (segment (start 131.125 92.725) (end 131.125 87.975) (width 0.25) (layer F.Cu) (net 17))
 (segment (start 133.15 93.5) (end 131.9 93.5) (width 0.25) (layer F.Cu) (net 17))
 (segment (start 112.85 98.275) (end 113.375 97.75) (width 0.25) (layer F.Cu) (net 13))
 (segment (start 112.85 100.2) (end 112.85 98.275) (width 0.25) (layer F.Cu) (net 13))
 (segment (start 139.475 86.6) (end 140.05 86.6) (width 0.25) (layer F.Cu) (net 12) (status 20))
 (segment (start 139 87.075) (end 139.475 86.6) (width 0.25) (layer F.Cu) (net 12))
 (segment (start 139 88.625) (end 139 87.075) (width 0.25) (layer F.Cu) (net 12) (status 10))
 (segment (start 139 88.625) (end 136.875 88.625) (width 0.25) (layer F.Cu) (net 12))
 (via (at 136.75 88.75) (size 0.8) (drill 0.4) (layers F.Cu B.Cu) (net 12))
 (segment (start 136.875 88.625) (end 136.75 88.75) (width 0.25) (layer F.Cu) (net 12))
 (segment (start 136.350001 89.149999) (end 122.600001 89.149999) (width 0.25) (layer B.Cu) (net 12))
 (segment (start 136.75 88.75) (end 136.350001 89.149999) (width 0.25) (layer B.Cu) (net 12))
 (via (at 117.5 94) (size 0.8) (drill 0.4) (layers F.Cu B.Cu) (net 12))
 (segment (start 122.600001 89.149999) (end 117.75 94) (width 0.25) (layer B.Cu) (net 12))
 (segment (start 117.75 94) (end 117.5 94) (width 0.25) (layer B.Cu) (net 12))
 (segment (start 115.65 97.75) (end 115.125 97.75) (width 0.25) (layer F.Cu) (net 12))
 (segment (start 117.5 95.9) (end 115.65 97.75) (width 0.25) (layer F.Cu) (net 12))
 (segment (start 117.5 94) (end 117.5 95.9) (width 0.25) (layer F.Cu) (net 12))
 (segment (start 142.525 90.375) (end 143 90.375) (width 0.25) (layer F.Cu) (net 10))
 (segment (start 141.95 89.8) (end 142.525 90.375) (width 0.25) (layer F.Cu) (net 10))
 (segment (start 141.95 86.6) (end 141.95 89.8) (width 0.25) (layer F.Cu) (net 10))
 (segment (start 140 90.375) (end 141 91.375) (width 0.25) (layer F.Cu) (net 10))
 (segment (start 139 90.375) (end 140 90.375) (width 0.25) (layer F.Cu) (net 10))
 (segment (start 142 90.375) (end 141 91.375) (width 0.25) (layer F.Cu) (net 10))
 (segment (start 143 90.375) (end 142 90.375) (width 0.25) (layer F.Cu) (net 10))
 (segment (start 159.9875 94) (end 159.9875 91) (width 1) (layer F.Cu) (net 7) (status 30))
 (segment (start 142 84.35) (end 141.95 84.4) (width 0.25) (layer F.Cu) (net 9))
 (segment (start 142 82.375) (end 142 84.35) (width 0.25) (layer F.Cu) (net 9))
 (segment (start 133.55 106.525) (end 132.325 107.75) (width 1) (layer F.Cu) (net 2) (status 10))
 (segment (start 134.25 106.525) (end 133.55 106.525) (width 1) (layer F.Cu) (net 2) (status 30))
 (via (at 148.5 97.25) (size 1.2) (drill 0.6) (layers F.Cu B.Cu) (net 2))
 (segment (start 150.25 96.45) (end 149.3 96.45) (width 1) (layer F.Cu) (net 2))
 (segment (start 149.3 96.45) (end 148.5 97.25) (width 1) (layer F.Cu) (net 2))
 (via (at 132.325 107.75) (size 1.2) (drill 0.6) (layers F.Cu B.Cu) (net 2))
 (segment (start 148.5 97.25) (end 138 107.75) (width 1) (layer B.Cu) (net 2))
 (via (at 105 102) (size 1.2) (drill 0.6) (layers F.Cu B.Cu) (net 2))
 (segment (start 135 107.75) (end 110.75 107.75) (width 1) (layer B.Cu) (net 2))
 (segment (start 138 107.75) (end 135 107.75) (width 1) (layer B.Cu) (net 2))
 (segment (start 135 107.75) (end 132.325 107.75) (width 1) (layer B.Cu) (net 2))
 (segment (start 105 101.1) (end 107 99.1) (width 1) (layer F.Cu) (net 2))
 (segment (start 105 102) (end 105 101.1) (width 1) (layer F.Cu) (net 2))
 (segment (start 106.5 103.5) (end 103 100) (width 1) (layer B.Cu) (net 2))
 (segment (start 110.75 107.75) (end 106.5 103.5) (width 1) (layer B.Cu) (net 2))
 (segment (start 106.5 103.5) (end 105 102) (width 1) (layer B.Cu) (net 2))
 (via (at 130.25 78.5) (size 1.2) (drill 0.6) (layers F.Cu B.Cu) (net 2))
 (segment (start 103 100) (end 97.75 100) (width 1) (layer B.Cu) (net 2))
 (segment (start 97.75 100) (end 95 100) (width 1) (layer B.Cu) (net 2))
 (segment (start 130.95 78.5) (end 132.65 80.2) (width 1) (layer F.Cu) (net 2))
 (segment (start 130.25 78.5) (end 130.95 78.5) (width 1) (layer F.Cu) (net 2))
 (segment (start 96.5 78.5) (end 130.25 78.5) (width 1) (layer B.Cu) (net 2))
 (segment (start 92.25 82.75) (end 96.5 78.5) (width 1) (layer B.Cu) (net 2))
 (segment (start 97.75 100) (end 92.25 94.5) (width 1) (layer B.Cu) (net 2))
 (segment (start 92.25 94.5) (end 92.25 82.75) (width 1) (layer B.Cu) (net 2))
 (via (at 101.25 90.75) (size 1.2) (drill 0.6) (layers F.Cu B.Cu) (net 11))
 (segment (start 99 90.975) (end 101.025 90.975) (width 1) (layer F.Cu) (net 11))
 (segment (start 101.025 90.975) (end 101.25 90.75) (width 1) (layer F.Cu) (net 11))
 (segment (start 130.25 83) (end 136 83) (width 1) (layer B.Cu) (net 11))
 (segment (start 136 83) (end 141 88) (width 1) (layer B.Cu) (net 11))
 (via (at 141 88) (size 1.2) (drill 0.6) (layers F.Cu B.Cu) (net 11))
 (segment (start 141 89.625) (end 141 88) (width 1) (layer F.Cu) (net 11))
 (segment (start 138.375 81.5) (end 137.5 81.5) (width 1) (layer F.Cu) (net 11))
 (via (at 136 83) (size 1.2) (drill 0.6) (layers F.Cu B.Cu) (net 11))
 (segment (start 137.5 81.5) (end 136 83) (width 1) (layer F.Cu) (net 11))
 (segment (start 132.65 82.5) (end 130.75 82.5) (width 1) (layer F.Cu) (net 11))
 (via (at 130.25 83) (size 1.2) (drill 0.6) (layers F.Cu B.Cu) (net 11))
 (segment (start 130.75 82.5) (end 130.25 83) (width 1) (layer F.Cu) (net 11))
 (segment (start 129.75 82.5) (end 130.25 83) (width 1) (layer F.Cu) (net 11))
 (segment (start 126.35 82.5) (end 129.75 82.5) (width 1) (layer F.Cu) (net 11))
 (segment (start 126.5 86.75) (end 130.25 83) (width 1) (layer F.Cu) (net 11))
 (segment (start 126.5 86.875) (end 126.5 86.75) (width 1) (layer F.Cu) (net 11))
 (segment (start 141 86.6) (end 141 88) (width 0.5) (layer F.Cu) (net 11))
 (segment (start 129 81.75) (end 130.25 83) (width 1) (layer B.Cu) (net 11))
 (segment (start 118 81.75) (end 129 81.75) (width 1) (layer B.Cu) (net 11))
 (segment (start 112.389999 87.360001) (end 118 81.75) (width 1) (layer B.Cu) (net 11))
 (segment (start 101.25 90.75) (end 104.639999 87.360001) (width 1) (layer B.Cu) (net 11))
 (segment (start 104.639999 87.360001) (end 112.389999 87.360001) (width 1) (layer B.Cu) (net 11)))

